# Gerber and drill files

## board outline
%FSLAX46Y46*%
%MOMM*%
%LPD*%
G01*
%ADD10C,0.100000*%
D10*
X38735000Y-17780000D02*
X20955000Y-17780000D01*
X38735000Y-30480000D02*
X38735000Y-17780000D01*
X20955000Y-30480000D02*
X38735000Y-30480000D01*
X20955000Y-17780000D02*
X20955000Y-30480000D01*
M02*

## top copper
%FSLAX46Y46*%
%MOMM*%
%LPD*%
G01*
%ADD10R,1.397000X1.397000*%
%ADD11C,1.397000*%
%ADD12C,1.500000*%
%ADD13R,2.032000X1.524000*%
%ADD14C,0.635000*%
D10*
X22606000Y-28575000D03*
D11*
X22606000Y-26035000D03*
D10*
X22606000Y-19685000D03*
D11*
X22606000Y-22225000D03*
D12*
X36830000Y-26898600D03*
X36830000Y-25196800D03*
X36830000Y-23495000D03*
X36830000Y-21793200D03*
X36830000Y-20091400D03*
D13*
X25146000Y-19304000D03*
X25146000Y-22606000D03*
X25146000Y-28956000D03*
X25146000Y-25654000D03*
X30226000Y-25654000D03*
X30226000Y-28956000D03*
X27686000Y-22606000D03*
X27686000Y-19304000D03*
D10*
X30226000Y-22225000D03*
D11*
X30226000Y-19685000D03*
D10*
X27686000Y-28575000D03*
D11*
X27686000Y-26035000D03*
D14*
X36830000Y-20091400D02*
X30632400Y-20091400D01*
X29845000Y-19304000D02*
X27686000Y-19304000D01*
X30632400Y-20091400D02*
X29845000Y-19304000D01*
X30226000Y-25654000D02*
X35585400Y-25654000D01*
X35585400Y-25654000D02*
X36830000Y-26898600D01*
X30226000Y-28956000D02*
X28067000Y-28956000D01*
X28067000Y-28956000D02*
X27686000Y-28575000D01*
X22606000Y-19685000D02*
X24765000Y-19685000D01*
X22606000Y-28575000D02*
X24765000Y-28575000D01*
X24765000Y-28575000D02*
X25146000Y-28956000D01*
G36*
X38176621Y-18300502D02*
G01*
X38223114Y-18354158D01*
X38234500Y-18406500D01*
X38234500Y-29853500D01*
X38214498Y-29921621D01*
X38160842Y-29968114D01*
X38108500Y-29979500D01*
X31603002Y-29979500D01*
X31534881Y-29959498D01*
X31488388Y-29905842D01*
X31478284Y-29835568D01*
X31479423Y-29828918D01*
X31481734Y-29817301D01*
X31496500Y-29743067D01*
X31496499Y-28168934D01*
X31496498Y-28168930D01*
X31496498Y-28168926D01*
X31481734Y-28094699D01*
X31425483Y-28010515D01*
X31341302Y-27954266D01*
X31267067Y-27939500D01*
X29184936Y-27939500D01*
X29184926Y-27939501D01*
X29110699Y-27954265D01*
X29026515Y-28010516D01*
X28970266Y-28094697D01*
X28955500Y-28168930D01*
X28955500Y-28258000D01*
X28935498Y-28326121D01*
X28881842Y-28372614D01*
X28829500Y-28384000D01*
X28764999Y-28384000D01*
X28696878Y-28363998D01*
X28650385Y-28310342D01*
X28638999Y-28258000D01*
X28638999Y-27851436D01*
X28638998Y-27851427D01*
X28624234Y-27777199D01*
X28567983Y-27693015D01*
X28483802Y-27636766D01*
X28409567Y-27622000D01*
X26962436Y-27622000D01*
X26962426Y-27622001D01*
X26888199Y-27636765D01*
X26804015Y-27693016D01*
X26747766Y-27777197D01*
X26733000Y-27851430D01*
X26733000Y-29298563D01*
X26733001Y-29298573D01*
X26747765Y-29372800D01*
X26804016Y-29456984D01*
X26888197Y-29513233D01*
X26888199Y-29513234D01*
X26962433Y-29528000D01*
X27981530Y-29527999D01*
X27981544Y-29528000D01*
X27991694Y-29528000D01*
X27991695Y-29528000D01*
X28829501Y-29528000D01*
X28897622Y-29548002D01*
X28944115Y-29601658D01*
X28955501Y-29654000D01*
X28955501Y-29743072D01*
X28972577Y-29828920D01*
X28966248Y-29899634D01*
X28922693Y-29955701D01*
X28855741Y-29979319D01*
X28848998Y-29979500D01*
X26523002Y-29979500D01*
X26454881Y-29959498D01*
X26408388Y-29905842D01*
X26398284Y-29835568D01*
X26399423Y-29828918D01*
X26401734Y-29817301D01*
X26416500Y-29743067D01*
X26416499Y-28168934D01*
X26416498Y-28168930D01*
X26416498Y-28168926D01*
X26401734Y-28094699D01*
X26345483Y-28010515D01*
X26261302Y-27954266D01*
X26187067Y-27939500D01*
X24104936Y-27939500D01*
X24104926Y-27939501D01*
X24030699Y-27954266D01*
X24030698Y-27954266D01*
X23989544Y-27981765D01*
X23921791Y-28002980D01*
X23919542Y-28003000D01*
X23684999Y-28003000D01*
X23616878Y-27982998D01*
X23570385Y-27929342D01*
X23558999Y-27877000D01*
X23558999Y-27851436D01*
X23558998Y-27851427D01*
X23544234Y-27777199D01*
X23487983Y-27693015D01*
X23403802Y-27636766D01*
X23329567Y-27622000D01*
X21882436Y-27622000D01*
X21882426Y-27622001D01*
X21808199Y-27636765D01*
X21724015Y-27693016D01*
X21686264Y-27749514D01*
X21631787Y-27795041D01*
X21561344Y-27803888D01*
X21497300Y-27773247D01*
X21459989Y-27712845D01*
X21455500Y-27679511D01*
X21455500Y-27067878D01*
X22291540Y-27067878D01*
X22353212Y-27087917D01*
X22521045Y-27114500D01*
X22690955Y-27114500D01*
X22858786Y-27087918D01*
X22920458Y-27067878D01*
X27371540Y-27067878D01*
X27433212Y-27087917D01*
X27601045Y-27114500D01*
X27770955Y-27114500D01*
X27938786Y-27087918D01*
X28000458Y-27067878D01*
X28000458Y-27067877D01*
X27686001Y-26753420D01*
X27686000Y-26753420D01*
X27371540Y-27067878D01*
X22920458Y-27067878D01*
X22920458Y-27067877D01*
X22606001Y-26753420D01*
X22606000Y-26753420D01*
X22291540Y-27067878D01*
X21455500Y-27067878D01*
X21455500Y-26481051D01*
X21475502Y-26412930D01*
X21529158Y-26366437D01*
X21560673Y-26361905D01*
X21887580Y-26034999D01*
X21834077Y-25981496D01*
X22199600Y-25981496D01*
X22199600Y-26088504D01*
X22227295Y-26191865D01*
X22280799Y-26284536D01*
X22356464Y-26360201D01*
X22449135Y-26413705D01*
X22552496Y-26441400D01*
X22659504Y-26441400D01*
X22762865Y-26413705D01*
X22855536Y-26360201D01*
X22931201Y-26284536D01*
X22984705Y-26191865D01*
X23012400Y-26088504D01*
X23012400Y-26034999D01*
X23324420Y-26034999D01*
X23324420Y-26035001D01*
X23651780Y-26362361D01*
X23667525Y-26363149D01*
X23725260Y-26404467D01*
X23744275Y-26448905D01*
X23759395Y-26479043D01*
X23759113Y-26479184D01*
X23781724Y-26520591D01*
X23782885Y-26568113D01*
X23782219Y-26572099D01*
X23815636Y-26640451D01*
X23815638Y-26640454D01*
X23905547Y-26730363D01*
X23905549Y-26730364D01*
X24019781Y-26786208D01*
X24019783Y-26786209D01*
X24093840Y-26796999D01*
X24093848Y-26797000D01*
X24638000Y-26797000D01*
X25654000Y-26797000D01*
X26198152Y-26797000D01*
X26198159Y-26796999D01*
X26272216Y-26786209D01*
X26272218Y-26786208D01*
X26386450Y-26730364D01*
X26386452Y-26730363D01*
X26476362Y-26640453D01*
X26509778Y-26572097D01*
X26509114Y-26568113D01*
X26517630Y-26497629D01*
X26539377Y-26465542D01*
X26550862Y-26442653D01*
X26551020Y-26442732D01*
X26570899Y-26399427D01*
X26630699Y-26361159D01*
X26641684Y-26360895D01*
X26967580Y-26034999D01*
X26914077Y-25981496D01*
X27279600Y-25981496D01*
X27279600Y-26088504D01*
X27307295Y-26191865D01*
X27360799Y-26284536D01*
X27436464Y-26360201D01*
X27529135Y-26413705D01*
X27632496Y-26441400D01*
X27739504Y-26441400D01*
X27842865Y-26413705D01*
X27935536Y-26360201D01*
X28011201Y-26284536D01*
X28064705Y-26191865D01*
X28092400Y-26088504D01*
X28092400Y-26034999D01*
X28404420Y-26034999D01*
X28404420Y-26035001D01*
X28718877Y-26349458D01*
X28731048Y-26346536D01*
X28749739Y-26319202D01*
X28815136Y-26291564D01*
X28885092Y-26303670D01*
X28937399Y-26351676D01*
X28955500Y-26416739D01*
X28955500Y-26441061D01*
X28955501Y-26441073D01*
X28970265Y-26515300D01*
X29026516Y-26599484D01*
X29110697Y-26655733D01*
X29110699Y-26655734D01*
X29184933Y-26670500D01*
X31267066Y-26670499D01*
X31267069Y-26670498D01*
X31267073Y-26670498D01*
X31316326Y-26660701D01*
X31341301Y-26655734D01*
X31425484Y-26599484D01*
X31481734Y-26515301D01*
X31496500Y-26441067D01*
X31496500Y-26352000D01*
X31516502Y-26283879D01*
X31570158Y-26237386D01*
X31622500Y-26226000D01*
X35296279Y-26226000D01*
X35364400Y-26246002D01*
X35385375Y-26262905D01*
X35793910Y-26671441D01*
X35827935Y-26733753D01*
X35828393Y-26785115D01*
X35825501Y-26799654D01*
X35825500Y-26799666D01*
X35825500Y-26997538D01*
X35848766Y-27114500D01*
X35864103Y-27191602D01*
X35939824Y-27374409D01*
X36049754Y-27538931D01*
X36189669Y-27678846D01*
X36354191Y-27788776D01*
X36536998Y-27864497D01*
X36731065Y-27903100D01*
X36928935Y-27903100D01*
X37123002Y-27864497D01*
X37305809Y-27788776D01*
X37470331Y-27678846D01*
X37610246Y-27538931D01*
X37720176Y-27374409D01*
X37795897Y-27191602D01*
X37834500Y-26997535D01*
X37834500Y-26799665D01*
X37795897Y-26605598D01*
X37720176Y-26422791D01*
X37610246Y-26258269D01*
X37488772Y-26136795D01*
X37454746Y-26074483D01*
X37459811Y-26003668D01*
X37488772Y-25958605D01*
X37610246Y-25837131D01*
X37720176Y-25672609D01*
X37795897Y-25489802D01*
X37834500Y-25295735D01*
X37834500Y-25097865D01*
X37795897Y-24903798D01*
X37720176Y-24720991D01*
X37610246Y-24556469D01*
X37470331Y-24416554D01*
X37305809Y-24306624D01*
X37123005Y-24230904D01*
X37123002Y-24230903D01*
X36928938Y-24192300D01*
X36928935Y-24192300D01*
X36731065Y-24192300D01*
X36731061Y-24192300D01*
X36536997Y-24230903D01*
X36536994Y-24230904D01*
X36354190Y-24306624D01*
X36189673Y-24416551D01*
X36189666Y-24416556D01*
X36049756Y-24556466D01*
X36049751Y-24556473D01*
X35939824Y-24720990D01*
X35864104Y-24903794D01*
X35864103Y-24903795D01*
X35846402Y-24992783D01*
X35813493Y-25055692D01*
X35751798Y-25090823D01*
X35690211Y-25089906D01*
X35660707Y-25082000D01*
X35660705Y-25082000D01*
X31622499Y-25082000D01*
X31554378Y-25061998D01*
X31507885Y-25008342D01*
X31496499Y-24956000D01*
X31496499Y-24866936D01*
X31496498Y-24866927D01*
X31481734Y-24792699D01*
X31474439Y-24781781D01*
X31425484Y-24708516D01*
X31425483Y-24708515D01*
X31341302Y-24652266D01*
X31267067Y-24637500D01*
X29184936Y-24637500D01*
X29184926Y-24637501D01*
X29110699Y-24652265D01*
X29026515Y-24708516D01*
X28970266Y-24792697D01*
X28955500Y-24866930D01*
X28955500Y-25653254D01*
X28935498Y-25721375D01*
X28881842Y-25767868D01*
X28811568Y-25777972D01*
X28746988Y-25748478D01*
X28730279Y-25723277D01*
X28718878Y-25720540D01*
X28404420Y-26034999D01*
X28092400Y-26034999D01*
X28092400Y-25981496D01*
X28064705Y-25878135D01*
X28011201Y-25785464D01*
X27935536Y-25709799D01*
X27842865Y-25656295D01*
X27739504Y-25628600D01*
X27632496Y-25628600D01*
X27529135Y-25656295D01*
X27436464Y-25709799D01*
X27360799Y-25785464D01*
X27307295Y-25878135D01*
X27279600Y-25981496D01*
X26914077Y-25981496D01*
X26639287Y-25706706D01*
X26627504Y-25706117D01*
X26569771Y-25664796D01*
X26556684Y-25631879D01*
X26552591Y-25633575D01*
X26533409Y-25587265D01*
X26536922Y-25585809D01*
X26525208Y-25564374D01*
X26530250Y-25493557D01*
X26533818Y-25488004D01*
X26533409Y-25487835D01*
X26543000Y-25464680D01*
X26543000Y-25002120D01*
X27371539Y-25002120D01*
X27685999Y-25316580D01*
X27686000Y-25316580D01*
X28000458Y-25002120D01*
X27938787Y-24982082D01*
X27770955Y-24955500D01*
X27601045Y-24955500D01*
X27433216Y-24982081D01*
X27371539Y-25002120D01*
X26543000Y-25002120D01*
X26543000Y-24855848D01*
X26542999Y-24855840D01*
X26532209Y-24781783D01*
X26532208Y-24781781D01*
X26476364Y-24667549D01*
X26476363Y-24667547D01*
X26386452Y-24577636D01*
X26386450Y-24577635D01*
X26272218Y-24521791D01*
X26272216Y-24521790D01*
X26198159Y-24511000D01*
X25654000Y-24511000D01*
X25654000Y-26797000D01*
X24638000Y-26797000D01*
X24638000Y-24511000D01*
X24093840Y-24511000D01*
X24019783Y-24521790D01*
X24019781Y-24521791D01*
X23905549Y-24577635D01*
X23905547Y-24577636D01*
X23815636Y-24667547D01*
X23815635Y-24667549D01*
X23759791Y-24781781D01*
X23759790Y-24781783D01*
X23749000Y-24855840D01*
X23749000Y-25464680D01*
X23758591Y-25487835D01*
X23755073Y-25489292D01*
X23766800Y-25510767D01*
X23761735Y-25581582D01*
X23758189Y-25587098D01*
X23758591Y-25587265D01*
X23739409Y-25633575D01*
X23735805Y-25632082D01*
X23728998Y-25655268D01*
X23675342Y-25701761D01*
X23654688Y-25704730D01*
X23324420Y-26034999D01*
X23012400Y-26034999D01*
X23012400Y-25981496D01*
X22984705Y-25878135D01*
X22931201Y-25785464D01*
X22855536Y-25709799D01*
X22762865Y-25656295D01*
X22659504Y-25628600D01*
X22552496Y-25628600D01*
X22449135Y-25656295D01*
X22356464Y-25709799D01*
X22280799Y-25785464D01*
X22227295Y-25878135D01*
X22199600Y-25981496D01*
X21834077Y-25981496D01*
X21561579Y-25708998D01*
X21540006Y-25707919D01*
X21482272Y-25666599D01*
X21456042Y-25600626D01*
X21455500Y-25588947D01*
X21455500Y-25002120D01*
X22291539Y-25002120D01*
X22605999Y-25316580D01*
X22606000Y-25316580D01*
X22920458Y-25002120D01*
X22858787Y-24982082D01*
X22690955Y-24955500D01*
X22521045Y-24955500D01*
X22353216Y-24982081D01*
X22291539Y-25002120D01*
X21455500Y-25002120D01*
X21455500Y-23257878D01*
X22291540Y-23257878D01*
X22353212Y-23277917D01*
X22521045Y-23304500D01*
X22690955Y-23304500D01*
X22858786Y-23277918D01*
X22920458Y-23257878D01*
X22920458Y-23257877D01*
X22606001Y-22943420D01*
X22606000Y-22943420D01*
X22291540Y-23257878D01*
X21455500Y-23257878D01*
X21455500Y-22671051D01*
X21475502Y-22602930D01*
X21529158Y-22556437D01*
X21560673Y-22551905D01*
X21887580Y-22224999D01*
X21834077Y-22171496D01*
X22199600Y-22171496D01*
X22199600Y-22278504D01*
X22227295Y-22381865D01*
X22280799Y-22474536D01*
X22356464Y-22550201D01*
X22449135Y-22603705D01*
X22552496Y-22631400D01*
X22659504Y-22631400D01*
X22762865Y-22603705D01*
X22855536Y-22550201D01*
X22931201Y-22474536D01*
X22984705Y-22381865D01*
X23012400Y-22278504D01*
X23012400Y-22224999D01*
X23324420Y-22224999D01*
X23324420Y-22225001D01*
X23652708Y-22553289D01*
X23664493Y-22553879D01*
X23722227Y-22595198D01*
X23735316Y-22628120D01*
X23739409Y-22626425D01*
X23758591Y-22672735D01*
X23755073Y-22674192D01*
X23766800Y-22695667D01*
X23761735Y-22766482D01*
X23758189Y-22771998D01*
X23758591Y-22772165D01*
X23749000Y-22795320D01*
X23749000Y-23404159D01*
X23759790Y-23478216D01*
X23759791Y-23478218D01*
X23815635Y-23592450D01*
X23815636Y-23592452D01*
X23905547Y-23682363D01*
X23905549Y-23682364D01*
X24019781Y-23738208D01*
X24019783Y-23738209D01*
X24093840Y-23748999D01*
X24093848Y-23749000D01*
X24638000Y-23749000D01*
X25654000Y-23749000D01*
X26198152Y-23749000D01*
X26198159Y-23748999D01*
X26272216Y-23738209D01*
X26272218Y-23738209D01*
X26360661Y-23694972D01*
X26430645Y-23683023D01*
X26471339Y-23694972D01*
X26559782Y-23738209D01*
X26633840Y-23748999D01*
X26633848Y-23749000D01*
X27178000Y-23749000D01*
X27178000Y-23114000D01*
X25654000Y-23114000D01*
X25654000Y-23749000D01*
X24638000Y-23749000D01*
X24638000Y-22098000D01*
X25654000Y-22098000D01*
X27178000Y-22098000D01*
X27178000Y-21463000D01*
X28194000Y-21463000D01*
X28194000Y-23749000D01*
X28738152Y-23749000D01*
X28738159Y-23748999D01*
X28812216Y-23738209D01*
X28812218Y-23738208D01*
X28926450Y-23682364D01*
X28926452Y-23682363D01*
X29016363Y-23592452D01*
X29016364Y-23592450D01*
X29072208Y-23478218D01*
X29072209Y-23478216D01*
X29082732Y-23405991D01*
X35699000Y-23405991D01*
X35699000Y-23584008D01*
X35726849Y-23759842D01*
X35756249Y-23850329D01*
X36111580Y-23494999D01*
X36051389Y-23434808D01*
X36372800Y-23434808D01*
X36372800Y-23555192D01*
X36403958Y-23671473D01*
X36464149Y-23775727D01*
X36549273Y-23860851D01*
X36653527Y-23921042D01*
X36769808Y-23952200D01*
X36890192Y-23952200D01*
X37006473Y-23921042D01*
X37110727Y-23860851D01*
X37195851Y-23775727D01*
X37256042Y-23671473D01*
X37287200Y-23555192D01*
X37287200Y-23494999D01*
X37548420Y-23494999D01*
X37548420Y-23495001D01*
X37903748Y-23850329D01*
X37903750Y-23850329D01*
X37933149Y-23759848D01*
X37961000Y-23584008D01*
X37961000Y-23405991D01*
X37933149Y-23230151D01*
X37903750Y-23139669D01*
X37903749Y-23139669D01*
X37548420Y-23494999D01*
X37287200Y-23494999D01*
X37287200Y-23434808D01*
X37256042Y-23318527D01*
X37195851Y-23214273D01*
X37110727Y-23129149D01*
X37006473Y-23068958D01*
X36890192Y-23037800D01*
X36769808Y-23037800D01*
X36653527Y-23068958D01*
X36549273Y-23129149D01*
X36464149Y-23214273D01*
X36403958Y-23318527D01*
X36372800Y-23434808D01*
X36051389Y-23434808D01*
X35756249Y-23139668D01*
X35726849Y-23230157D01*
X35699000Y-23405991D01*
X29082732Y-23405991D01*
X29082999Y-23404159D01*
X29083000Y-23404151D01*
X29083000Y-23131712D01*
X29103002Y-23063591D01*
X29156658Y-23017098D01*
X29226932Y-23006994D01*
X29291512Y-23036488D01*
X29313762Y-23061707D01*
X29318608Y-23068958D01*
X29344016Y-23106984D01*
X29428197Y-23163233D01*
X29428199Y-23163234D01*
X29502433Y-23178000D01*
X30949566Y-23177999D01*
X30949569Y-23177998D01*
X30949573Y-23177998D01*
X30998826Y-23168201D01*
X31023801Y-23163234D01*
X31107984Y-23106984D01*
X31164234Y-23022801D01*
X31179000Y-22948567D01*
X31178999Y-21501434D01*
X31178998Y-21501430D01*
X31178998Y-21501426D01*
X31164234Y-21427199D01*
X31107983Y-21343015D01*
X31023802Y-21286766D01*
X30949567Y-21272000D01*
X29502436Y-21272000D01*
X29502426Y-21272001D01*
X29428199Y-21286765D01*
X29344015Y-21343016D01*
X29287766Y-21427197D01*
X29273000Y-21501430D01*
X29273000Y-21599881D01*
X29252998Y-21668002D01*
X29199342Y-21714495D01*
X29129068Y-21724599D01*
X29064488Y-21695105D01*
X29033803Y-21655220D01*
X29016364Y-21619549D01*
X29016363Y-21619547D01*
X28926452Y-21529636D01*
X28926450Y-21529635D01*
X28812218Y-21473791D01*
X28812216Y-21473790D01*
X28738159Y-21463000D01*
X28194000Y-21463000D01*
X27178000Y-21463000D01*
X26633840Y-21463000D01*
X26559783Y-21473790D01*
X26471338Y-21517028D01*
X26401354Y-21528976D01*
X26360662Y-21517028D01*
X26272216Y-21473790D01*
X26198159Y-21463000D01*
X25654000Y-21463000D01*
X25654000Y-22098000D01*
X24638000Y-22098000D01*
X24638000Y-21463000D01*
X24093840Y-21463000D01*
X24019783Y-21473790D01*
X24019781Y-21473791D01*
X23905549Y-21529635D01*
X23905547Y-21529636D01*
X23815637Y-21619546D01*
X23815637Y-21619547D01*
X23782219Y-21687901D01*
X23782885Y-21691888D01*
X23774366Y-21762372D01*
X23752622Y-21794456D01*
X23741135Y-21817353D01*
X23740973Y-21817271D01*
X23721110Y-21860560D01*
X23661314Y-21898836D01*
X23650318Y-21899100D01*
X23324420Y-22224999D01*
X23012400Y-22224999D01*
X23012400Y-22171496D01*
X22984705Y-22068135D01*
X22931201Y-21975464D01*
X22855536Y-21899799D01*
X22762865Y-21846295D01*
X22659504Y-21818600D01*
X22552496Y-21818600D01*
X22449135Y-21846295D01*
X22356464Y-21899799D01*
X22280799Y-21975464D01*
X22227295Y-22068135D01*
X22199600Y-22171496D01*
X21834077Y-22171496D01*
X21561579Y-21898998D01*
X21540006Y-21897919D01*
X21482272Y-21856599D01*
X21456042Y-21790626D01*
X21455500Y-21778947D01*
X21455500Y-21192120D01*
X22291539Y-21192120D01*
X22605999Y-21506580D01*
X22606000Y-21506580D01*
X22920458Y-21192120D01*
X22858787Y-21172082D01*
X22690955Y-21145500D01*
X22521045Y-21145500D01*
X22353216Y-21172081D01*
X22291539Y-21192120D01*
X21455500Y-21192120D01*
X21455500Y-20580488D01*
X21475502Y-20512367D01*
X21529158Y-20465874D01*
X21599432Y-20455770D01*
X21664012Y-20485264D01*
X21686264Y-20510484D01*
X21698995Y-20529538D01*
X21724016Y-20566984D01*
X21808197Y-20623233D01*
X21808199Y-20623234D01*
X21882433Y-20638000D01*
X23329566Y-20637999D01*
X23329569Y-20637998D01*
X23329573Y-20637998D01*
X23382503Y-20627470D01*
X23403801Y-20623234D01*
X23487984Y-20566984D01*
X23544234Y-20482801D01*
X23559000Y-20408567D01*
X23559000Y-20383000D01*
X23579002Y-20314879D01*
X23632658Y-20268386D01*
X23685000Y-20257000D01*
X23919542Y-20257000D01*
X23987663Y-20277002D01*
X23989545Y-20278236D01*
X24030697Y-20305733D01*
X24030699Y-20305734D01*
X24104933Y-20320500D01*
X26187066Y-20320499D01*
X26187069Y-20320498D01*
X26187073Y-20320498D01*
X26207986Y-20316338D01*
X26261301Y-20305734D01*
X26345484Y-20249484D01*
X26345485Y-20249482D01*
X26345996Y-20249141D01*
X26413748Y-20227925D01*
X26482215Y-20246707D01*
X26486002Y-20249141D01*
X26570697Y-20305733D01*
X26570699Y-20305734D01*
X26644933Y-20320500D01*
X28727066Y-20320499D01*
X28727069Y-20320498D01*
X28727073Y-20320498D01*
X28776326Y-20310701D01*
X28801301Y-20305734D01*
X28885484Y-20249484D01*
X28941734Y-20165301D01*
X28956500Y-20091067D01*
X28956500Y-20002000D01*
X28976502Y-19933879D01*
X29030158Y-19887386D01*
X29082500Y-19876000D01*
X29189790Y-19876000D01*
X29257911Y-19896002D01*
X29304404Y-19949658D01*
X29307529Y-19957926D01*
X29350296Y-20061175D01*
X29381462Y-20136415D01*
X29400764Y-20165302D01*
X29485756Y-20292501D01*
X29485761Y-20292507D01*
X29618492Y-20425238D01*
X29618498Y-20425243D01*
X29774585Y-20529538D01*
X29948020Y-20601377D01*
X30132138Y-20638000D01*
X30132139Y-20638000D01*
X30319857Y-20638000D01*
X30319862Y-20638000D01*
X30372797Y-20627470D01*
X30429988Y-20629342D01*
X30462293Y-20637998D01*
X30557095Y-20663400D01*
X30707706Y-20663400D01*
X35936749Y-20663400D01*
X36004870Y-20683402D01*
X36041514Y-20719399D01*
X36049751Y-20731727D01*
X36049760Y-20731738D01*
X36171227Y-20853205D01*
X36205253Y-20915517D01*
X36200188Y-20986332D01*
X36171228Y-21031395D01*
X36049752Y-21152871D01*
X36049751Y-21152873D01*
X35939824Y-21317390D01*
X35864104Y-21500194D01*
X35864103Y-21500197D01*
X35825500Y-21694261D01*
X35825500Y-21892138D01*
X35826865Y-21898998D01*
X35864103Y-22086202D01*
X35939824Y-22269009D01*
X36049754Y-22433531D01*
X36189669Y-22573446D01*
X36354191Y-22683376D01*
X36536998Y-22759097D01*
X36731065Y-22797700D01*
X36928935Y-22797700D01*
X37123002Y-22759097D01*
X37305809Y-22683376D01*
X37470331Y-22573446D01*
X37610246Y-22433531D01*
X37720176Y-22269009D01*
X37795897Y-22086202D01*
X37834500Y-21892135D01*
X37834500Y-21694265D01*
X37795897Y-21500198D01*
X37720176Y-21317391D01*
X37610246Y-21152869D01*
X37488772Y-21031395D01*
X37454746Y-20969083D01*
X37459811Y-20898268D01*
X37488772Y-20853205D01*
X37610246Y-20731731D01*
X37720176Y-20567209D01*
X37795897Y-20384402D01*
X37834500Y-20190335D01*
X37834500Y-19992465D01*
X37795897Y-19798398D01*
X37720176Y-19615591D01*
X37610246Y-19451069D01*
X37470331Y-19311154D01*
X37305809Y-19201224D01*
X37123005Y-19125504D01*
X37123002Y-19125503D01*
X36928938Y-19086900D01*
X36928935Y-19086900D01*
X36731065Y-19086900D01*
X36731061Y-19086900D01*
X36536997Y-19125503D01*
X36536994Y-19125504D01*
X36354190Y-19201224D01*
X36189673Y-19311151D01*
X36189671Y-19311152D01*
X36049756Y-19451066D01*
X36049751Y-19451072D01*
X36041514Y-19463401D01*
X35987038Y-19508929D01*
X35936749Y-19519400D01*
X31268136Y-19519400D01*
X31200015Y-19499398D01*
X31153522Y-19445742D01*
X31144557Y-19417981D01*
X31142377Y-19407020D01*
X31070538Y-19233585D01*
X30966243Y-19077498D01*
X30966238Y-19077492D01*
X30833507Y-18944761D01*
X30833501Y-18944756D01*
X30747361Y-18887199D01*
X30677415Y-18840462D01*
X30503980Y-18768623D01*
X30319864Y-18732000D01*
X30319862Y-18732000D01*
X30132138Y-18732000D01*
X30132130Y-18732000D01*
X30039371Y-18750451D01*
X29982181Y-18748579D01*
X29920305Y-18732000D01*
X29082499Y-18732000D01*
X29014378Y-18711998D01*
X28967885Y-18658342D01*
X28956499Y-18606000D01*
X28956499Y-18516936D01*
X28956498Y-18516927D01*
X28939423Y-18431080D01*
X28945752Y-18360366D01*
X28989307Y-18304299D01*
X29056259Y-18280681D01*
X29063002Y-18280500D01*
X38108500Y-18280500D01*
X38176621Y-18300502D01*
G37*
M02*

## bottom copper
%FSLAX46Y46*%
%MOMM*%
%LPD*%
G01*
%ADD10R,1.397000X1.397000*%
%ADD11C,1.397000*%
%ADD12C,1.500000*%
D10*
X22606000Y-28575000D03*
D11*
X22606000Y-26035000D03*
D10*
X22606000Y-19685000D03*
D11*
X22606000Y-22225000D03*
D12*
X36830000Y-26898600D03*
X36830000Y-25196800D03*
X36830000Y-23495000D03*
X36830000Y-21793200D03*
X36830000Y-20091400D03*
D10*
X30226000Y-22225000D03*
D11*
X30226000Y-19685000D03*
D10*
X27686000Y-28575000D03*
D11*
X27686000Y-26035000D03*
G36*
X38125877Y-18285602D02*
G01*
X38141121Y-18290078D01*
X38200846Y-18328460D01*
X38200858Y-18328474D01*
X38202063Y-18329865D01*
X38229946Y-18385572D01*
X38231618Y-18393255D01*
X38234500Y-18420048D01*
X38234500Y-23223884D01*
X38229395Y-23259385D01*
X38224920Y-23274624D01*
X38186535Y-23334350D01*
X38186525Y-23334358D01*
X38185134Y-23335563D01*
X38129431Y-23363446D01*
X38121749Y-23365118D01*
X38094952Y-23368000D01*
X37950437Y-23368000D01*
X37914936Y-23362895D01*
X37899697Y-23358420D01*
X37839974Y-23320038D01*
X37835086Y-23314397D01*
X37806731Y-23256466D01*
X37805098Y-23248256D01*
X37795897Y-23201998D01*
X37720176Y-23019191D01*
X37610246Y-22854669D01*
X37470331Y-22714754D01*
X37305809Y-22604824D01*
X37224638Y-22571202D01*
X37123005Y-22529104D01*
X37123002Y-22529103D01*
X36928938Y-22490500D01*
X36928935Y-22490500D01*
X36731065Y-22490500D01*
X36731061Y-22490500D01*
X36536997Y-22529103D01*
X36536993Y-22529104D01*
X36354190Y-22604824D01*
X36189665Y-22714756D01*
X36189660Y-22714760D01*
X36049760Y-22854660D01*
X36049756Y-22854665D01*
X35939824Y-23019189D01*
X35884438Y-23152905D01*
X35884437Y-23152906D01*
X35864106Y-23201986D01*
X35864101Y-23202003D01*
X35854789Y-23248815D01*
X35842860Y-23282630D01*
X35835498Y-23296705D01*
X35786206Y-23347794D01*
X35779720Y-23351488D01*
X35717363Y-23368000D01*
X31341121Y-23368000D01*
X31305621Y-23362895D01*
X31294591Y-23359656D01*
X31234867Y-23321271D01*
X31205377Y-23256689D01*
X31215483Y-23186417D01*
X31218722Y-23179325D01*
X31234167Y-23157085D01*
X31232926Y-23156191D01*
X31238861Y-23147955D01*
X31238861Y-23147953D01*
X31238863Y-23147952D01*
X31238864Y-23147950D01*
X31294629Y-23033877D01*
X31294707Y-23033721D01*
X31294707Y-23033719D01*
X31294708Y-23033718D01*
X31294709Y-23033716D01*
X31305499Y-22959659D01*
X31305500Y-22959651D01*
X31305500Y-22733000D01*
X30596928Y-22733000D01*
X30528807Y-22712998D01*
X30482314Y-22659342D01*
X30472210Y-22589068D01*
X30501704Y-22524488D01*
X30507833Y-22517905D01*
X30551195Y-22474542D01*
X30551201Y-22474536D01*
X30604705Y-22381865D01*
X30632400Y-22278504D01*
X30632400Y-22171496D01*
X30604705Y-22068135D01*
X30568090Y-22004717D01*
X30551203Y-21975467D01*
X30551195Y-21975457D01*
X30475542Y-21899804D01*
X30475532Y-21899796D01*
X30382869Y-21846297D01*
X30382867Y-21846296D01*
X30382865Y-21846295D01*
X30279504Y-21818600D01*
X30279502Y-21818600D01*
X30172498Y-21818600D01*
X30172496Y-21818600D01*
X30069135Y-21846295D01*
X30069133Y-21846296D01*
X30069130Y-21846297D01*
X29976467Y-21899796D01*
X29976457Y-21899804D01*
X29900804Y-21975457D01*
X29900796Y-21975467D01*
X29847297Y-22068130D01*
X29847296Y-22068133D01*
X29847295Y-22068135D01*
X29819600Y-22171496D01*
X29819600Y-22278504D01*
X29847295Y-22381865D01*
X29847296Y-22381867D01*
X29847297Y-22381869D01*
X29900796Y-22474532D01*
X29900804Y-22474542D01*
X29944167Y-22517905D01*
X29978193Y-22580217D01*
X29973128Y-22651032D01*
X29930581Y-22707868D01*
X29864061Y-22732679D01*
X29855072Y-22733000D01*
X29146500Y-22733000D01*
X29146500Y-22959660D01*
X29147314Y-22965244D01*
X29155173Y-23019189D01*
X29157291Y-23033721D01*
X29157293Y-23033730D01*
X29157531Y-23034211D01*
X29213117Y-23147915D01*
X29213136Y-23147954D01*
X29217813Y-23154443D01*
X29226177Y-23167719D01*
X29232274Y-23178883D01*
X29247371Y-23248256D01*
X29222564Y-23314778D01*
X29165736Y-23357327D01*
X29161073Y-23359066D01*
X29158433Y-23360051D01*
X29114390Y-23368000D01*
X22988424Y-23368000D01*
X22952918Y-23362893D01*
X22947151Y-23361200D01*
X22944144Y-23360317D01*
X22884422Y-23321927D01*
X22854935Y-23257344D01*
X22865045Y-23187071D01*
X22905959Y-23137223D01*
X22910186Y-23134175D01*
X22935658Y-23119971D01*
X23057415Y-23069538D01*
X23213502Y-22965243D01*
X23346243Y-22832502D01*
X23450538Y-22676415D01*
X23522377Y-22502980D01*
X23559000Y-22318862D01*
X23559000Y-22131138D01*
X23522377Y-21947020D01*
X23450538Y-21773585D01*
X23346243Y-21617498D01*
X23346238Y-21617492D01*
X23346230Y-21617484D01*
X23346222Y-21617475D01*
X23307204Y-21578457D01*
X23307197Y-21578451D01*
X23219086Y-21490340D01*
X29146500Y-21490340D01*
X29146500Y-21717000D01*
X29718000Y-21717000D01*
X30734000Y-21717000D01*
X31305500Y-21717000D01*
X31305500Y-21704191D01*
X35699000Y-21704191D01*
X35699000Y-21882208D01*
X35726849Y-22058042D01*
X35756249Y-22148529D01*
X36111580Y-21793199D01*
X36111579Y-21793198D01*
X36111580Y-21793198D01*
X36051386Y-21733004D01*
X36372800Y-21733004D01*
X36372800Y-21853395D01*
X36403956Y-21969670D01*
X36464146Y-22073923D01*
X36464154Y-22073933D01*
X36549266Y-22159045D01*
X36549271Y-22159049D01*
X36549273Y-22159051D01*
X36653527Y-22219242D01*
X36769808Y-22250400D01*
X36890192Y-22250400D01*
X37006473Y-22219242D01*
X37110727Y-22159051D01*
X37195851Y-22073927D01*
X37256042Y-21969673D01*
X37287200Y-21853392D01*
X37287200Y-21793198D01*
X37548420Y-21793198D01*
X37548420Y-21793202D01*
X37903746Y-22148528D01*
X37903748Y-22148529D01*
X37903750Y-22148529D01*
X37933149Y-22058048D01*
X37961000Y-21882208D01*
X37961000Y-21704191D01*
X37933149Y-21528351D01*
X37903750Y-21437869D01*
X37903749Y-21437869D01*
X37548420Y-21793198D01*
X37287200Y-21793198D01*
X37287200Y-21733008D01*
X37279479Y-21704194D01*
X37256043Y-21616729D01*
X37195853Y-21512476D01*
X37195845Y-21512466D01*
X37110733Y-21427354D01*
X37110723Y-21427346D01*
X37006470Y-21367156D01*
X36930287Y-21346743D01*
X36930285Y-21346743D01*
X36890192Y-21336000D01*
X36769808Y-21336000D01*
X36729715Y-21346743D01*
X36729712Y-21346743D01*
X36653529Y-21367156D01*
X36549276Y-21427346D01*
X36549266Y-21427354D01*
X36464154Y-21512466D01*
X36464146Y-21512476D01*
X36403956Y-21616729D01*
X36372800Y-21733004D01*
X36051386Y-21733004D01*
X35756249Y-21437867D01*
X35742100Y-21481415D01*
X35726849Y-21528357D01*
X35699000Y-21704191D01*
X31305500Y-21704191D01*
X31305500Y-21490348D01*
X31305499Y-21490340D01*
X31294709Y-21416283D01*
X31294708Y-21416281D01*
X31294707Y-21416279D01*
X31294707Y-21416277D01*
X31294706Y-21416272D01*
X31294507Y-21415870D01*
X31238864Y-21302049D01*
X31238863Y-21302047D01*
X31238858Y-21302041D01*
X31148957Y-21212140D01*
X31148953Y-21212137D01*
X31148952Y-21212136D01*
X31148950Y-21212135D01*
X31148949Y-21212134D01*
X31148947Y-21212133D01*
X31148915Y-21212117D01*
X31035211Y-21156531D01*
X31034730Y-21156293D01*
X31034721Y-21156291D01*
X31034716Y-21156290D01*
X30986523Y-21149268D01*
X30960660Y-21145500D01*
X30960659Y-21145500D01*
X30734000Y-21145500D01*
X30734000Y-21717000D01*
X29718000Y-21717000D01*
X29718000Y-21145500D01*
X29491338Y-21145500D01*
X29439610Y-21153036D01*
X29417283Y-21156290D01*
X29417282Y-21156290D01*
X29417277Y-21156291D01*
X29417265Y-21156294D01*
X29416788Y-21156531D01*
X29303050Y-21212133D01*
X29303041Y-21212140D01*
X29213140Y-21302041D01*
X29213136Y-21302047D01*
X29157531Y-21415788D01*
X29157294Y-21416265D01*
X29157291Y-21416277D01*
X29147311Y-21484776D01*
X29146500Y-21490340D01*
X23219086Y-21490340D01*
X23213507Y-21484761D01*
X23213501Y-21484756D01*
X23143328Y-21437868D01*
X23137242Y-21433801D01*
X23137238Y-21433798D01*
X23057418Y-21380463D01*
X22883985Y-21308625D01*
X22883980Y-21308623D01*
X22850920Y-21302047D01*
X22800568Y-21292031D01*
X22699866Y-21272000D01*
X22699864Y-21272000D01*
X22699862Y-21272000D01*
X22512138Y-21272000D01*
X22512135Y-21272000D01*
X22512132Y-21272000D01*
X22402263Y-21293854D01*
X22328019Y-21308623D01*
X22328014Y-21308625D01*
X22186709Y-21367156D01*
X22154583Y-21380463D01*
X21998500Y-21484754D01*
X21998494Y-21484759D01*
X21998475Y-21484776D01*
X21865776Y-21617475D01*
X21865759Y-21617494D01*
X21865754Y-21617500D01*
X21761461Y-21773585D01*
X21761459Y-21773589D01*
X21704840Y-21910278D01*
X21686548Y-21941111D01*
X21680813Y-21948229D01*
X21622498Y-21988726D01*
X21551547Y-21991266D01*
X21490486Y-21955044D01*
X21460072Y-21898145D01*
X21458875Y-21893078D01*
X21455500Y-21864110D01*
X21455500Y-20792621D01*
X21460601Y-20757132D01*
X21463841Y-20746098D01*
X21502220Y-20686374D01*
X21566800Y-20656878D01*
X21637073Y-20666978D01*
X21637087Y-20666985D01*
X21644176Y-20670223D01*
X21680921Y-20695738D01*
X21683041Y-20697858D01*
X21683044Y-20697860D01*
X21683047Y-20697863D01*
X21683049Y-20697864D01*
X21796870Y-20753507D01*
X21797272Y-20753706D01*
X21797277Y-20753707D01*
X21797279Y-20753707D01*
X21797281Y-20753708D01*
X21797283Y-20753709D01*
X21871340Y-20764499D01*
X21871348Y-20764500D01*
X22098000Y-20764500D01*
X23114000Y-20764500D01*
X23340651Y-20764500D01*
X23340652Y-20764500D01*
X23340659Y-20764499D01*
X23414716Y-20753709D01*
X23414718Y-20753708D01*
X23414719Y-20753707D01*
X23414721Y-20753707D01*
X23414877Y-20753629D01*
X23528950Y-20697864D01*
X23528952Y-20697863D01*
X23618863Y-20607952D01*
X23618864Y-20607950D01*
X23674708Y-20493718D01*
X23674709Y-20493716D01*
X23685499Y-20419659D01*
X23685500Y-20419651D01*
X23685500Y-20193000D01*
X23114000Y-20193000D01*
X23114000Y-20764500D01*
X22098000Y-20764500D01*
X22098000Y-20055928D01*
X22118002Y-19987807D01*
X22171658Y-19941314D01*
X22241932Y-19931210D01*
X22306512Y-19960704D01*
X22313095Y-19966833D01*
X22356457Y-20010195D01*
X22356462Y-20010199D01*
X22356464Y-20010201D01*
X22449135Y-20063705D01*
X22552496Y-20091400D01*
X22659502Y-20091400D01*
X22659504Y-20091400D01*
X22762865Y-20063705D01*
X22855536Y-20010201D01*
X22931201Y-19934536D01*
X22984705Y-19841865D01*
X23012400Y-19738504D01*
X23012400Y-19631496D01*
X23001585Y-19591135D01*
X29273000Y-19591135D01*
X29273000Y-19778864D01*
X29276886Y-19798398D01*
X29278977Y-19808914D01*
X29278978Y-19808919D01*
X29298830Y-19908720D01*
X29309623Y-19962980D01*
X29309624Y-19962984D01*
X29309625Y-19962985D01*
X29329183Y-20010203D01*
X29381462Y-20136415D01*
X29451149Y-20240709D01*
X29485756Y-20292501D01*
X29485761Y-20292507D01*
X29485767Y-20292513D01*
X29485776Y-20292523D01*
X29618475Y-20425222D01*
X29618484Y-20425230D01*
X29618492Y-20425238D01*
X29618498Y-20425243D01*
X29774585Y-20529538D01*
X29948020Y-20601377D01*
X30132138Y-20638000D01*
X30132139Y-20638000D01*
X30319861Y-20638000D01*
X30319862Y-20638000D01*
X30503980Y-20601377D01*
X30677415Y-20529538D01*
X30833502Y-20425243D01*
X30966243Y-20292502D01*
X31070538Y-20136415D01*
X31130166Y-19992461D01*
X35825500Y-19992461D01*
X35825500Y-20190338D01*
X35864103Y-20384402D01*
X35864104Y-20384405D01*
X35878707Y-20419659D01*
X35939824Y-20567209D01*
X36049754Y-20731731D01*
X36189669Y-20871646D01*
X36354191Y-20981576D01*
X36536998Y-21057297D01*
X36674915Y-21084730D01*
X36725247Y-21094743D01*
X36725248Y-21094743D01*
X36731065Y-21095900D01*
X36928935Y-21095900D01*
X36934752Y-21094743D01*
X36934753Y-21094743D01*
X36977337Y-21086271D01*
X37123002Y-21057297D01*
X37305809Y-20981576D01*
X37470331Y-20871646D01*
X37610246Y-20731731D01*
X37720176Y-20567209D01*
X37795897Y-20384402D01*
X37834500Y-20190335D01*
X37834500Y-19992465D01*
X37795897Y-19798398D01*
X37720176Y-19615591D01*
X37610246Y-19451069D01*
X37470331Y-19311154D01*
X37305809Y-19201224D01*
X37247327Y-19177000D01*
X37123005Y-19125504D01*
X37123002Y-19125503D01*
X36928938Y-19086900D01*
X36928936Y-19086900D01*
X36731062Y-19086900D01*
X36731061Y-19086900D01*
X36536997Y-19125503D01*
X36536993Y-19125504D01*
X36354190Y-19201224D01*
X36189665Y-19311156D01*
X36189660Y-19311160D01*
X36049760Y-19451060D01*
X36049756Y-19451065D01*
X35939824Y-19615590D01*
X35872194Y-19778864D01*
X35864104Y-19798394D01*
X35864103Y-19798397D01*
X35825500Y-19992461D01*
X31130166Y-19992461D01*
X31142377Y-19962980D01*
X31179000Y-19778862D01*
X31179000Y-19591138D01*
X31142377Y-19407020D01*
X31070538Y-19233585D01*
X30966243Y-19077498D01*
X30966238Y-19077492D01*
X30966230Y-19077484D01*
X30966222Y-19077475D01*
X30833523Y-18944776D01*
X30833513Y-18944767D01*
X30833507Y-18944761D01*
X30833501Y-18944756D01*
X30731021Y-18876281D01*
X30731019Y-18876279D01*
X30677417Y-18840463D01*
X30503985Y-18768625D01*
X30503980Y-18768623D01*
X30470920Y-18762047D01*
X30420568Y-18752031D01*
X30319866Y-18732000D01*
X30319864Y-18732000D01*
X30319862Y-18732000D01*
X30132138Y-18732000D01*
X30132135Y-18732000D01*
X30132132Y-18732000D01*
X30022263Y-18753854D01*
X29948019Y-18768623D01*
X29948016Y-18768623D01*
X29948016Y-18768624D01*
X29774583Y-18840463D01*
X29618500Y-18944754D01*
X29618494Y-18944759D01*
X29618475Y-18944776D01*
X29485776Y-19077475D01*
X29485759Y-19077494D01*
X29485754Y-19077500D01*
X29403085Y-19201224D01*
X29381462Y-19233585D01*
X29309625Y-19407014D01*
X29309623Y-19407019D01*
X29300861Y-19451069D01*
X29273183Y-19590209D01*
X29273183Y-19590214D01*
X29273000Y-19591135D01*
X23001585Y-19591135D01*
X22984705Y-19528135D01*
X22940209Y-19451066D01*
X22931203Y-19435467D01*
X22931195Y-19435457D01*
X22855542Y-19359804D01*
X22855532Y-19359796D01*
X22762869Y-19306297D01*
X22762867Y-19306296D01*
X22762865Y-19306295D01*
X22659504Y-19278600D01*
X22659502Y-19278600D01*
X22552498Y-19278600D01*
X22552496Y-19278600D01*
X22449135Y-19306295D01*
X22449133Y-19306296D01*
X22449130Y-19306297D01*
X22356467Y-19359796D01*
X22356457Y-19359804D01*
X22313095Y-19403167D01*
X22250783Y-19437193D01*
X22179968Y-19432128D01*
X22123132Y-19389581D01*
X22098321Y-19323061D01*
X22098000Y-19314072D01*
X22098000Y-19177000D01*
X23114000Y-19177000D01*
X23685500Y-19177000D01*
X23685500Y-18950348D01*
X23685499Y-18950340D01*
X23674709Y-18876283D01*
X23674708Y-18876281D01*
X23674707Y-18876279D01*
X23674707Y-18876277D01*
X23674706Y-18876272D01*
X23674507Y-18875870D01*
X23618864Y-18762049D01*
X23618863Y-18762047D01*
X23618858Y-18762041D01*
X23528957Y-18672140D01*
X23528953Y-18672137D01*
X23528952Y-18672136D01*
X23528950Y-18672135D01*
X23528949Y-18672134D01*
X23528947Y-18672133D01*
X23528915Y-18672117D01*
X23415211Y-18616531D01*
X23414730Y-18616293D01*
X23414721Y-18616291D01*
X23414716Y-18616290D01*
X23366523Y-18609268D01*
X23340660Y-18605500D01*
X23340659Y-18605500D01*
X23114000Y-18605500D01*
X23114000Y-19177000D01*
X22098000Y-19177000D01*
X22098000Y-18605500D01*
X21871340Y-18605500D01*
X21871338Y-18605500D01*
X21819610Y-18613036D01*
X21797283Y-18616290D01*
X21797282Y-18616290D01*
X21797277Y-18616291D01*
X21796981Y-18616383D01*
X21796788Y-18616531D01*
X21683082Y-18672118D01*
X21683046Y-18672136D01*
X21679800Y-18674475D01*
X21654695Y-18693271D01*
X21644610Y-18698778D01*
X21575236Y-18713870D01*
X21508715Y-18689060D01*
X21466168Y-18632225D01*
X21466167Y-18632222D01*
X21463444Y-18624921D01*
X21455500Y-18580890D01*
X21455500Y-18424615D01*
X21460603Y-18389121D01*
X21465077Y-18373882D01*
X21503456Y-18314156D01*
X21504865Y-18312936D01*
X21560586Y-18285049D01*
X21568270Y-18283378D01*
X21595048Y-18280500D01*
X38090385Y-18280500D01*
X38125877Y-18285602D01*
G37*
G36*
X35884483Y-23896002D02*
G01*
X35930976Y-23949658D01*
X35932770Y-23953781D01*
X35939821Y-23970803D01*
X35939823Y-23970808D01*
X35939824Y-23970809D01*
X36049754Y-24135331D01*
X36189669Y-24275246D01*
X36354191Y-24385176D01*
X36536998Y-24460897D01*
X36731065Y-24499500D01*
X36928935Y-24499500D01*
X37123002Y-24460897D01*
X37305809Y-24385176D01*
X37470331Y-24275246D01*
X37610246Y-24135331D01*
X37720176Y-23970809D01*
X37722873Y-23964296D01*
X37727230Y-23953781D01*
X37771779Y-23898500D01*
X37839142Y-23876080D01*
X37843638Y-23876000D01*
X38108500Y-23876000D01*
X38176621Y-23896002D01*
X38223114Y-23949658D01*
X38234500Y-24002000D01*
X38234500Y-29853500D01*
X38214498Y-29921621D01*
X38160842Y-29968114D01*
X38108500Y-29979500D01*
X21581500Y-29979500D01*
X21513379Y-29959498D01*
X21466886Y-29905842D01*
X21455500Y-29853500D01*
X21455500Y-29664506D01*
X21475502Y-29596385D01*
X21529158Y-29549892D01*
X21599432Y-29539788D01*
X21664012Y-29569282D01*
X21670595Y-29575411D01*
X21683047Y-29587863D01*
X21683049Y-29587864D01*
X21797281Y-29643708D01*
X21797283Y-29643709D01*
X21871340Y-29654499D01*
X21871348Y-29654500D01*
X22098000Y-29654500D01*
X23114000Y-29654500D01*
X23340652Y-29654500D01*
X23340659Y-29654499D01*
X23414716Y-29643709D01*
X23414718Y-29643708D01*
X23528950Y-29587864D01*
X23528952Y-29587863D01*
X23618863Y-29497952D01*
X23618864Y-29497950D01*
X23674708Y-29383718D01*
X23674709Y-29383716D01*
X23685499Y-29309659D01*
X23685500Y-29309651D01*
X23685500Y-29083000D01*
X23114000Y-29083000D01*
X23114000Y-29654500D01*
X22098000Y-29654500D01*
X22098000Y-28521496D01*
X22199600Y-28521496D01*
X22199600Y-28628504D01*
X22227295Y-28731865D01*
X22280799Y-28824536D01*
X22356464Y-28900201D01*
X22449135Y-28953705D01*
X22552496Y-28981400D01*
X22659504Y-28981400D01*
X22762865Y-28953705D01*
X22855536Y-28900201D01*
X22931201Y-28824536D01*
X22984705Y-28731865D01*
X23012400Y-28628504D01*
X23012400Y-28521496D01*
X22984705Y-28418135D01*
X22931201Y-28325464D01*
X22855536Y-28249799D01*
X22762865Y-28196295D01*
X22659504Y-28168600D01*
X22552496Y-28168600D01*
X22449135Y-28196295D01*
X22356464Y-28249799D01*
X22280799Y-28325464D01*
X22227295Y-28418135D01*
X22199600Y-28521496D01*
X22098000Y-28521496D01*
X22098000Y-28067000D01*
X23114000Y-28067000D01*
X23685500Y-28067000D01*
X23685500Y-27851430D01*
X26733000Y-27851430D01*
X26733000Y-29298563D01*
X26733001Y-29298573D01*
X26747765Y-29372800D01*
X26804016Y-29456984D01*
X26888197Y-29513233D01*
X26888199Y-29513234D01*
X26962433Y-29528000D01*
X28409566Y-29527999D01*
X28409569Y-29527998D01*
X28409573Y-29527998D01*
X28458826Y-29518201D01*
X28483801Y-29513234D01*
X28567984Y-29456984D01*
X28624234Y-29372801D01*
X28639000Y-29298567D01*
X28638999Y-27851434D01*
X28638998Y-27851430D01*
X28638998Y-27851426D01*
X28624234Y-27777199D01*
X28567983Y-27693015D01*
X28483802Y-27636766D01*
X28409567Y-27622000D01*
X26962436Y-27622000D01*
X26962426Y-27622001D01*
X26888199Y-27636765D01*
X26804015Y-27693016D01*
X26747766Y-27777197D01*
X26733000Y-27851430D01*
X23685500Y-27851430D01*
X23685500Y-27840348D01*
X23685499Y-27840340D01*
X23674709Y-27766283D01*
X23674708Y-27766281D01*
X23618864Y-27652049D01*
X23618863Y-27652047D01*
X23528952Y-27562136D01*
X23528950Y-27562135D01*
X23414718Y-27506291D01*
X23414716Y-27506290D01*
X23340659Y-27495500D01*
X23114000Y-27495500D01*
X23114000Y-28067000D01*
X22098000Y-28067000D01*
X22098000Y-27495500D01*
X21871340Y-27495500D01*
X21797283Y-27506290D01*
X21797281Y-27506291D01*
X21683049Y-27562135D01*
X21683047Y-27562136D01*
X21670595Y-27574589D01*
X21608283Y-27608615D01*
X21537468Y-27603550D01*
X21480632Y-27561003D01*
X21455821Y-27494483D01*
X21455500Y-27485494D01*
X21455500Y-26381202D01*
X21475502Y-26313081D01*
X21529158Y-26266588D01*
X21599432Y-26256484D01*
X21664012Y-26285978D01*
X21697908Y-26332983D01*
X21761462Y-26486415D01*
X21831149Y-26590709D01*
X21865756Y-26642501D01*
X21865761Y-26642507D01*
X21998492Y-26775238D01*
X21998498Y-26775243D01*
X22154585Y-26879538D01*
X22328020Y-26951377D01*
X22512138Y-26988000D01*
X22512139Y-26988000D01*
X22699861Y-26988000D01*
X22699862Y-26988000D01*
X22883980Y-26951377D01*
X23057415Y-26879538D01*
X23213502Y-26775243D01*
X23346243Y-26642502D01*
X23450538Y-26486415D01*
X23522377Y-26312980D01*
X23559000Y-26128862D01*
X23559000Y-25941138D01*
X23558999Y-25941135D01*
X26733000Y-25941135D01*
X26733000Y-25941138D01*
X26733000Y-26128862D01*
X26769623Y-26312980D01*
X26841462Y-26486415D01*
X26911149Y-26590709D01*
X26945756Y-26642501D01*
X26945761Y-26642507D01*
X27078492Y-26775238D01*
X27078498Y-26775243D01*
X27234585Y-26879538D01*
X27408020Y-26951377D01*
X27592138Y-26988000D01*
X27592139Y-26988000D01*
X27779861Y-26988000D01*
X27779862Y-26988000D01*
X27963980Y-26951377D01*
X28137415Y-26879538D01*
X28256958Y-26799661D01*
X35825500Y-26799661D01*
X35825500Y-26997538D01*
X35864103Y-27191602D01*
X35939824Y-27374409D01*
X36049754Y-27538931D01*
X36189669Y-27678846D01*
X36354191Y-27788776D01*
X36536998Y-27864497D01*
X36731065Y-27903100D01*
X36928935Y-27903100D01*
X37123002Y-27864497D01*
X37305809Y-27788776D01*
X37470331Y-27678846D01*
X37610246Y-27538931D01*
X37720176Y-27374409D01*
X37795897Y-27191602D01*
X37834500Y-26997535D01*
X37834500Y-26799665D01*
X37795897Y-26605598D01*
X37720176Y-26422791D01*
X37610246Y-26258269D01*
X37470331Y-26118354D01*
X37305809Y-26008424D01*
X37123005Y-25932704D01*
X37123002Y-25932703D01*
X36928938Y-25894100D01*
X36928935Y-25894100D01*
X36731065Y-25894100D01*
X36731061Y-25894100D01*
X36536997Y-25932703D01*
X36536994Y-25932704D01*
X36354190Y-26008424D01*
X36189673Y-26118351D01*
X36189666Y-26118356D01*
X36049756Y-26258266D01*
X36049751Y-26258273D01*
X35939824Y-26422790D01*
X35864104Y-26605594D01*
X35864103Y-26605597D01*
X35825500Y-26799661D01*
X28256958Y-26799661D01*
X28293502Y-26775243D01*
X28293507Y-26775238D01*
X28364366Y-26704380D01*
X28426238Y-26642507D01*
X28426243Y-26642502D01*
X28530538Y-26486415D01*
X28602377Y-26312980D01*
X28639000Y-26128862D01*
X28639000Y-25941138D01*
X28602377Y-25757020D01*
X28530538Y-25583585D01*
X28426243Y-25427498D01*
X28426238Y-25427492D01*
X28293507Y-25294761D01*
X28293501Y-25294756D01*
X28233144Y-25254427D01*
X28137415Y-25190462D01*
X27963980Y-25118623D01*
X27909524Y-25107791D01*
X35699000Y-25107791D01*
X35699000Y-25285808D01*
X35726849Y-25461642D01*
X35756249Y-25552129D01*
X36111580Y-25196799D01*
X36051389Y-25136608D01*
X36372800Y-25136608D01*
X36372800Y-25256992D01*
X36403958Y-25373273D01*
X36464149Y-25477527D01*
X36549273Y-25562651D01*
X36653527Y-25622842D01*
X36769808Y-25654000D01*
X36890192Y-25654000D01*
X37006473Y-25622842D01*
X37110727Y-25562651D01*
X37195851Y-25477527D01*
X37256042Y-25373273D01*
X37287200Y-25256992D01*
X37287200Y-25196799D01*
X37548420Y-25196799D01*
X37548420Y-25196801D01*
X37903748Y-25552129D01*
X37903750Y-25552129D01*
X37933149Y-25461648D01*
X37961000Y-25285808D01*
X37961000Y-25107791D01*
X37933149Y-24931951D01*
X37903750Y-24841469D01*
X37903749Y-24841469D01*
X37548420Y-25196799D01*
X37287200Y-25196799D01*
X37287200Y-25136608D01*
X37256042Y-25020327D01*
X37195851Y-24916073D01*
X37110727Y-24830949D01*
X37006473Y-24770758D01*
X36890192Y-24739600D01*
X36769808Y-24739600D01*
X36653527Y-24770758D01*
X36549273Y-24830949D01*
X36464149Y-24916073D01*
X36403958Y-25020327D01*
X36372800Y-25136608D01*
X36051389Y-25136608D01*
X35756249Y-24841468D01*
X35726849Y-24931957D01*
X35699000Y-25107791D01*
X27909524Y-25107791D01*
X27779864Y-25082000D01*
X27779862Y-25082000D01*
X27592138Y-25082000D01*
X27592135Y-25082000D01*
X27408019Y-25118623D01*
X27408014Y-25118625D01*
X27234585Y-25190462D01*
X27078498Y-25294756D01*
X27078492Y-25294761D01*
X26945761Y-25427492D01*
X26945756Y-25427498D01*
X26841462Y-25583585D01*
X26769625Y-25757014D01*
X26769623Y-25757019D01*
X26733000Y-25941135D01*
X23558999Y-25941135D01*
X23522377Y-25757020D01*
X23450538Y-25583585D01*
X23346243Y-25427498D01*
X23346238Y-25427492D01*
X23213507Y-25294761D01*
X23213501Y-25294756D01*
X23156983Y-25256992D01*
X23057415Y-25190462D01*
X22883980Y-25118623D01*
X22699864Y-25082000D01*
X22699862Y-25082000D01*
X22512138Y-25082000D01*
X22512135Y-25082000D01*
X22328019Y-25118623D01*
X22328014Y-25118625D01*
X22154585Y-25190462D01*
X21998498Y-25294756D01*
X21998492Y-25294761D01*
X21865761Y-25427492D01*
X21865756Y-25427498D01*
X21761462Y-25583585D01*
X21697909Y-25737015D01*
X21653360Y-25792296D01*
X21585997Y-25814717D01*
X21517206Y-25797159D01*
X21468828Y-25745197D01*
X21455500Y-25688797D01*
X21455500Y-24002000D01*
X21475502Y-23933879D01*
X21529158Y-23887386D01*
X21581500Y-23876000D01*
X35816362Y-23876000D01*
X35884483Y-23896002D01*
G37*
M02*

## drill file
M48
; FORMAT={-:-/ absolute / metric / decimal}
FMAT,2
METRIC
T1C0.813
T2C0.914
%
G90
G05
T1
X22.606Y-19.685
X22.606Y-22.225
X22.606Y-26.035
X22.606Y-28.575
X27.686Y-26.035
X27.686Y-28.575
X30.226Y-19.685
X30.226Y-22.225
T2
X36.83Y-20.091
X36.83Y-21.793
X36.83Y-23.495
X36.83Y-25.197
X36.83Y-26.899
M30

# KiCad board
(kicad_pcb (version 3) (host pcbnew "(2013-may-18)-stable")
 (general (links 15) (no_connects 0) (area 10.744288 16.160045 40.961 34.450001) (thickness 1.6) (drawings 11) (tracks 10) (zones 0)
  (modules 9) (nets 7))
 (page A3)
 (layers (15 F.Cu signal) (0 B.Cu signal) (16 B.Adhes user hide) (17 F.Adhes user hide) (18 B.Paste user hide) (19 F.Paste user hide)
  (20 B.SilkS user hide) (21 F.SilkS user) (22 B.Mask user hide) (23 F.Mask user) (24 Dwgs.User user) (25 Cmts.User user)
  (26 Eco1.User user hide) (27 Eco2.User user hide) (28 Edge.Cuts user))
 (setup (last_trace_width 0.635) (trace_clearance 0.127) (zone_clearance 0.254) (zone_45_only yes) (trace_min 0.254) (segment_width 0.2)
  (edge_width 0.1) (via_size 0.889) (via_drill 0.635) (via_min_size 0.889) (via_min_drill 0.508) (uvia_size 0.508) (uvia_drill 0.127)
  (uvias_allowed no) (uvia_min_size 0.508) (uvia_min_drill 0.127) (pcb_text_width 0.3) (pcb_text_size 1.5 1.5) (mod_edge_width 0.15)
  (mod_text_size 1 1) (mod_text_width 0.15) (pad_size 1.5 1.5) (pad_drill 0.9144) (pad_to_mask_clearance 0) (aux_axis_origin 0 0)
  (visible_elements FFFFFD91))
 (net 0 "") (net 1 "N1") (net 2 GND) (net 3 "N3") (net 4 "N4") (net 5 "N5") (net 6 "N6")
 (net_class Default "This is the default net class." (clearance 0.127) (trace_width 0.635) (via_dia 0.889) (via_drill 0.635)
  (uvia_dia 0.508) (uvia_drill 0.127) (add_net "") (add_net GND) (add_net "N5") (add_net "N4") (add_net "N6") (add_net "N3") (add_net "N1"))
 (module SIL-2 (layer F.Cu) (at 22.606 27.305 90)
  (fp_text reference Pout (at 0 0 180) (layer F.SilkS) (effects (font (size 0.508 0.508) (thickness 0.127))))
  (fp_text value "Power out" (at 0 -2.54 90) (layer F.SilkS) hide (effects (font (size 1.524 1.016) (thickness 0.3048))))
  (pad 1 thru_hole rect (at -1.27 0 90) (size 1.397 1.397) (drill 0.8128) (layers *.Cu *.Mask F.SilkS) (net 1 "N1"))
  (pad 2 thru_hole circle (at 1.27 0 90) (size 1.397 1.397) (drill 0.8128) (layers *.Cu *.Mask F.SilkS) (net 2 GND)))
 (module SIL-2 (layer F.Cu) (at 22.606 20.955 270)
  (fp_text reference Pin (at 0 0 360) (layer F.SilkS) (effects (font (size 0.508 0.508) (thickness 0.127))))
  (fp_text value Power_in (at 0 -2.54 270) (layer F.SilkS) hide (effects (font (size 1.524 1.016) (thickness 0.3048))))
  (pad 1 thru_hole rect (at -1.27 0 270) (size 1.397 1.397) (drill 0.8128) (layers *.Cu *.Mask F.SilkS) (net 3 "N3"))
  (pad 2 thru_hole circle (at 1.27 0 270) (size 1.397 1.397) (drill 0.8128) (layers *.Cu *.Mask F.SilkS) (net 2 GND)))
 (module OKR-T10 (layer F.Cu) (at 36.83 23.495 90)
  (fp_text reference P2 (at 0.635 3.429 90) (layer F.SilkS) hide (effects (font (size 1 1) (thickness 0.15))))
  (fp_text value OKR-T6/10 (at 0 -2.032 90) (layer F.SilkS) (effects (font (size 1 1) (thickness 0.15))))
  (pad 5 thru_hole circle (at -3.4036 0 90) (size 1.5 1.5) (drill 0.9144) (layers *.Cu *.Mask F.SilkS) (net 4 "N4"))
  (pad 4 thru_hole circle (at -1.7018 0 90) (size 1.5 1.5) (drill 0.9144) (layers *.Cu *.Mask F.SilkS) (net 1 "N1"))
  (pad 3 thru_hole circle (at 0 0 90) (size 1.5 1.5) (drill 0.9144) (layers *.Cu *.Mask F.SilkS) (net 2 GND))
  (pad 2 thru_hole circle (at 1.7018 0 90) (size 1.5 1.5) (drill 0.9144) (layers *.Cu *.Mask F.SilkS) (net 3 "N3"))
  (pad 1 thru_hole circle (at 3.4036 0 90) (size 1.5 1.5) (drill 0.9144) (layers *.Cu *.Mask F.SilkS) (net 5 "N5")))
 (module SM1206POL (layer F.Cu) (at 25.146 20.955 270)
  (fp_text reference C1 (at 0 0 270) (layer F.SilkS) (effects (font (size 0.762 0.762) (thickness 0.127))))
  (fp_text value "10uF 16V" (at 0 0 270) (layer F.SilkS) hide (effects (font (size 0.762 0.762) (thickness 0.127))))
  (pad 1 smd rect (at -1.651 0 270) (size 1.524 2.032) (layers F.Cu F.Paste F.Mask) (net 3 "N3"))
  (pad 2 smd rect (at 1.651 0 270) (size 1.524 2.032) (layers F.Cu F.Paste F.Mask) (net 2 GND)))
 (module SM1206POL (layer F.Cu) (at 25.146 27.305 90)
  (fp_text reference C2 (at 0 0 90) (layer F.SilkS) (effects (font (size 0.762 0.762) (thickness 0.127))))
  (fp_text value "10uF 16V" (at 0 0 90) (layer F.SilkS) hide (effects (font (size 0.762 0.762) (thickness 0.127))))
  (pad 1 smd rect (at -1.651 0 90) (size 1.524 2.032) (layers F.Cu F.Paste F.Mask) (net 1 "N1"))
  (pad 2 smd rect (at 1.651 0 90) (size 1.524 2.032) (layers F.Cu F.Paste F.Mask) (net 2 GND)))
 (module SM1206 (layer F.Cu) (at 30.226 27.305 270)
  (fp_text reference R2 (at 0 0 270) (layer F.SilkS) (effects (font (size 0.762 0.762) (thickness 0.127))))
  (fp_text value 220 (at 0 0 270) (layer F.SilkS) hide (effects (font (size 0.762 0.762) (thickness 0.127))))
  (pad 1 smd rect (at -1.651 0 270) (size 1.524 2.032) (layers F.Cu F.Paste F.Mask) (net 4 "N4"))
  (pad 2 smd rect (at 1.651 0 270) (size 1.524 2.032) (layers F.Cu F.Paste F.Mask) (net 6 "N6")))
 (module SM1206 (layer F.Cu) (at 27.686 20.955 90)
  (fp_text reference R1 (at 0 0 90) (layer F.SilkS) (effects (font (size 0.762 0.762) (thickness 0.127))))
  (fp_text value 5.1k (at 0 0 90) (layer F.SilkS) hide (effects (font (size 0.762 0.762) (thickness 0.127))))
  (pad 1 smd rect (at -1.651 0 90) (size 1.524 2.032) (layers F.Cu F.Paste F.Mask) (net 2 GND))
  (pad 2 smd rect (at 1.651 0 90) (size 1.524 2.032) (layers F.Cu F.Paste F.Mask) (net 5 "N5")))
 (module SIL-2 (layer F.Cu) (at 30.226 20.955 90)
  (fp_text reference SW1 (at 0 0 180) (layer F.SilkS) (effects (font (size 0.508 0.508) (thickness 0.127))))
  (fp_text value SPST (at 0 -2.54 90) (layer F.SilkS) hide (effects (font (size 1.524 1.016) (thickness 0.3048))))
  (pad 1 thru_hole rect (at -1.27 0 90) (size 1.397 1.397) (drill 0.8128) (layers *.Cu *.Mask F.SilkS) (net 3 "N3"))
  (pad 2 thru_hole circle (at 1.27 0 90) (size 1.397 1.397) (drill 0.8128) (layers *.Cu *.Mask F.SilkS) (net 5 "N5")))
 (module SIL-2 (layer F.Cu) (at 27.686 27.305 90)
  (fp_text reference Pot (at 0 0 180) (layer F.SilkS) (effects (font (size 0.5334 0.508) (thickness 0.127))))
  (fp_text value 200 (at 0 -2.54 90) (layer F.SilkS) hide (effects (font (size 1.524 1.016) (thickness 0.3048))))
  (pad 1 thru_hole rect (at -1.27 0 90) (size 1.397 1.397) (drill 0.8128) (layers *.Cu *.Mask F.SilkS) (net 6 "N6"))
  (pad 2 thru_hole circle (at 1.27 0 90) (size 1.397 1.397) (drill 0.8128) (layers *.Cu *.Mask F.SilkS) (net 2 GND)))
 (gr_line (start 38.735 17.78) (end 20.955 17.78) (angle 90) (layer Edge.Cuts) (width 0.1))
 (gr_line (start 38.735 30.48) (end 38.735 17.78) (angle 90) (layer Edge.Cuts) (width 0.1))
 (gr_line (start 20.955 30.48) (end 38.735 30.48) (angle 90) (layer Edge.Cuts) (width 0.1))
 (gr_line (start 20.955 17.78) (end 20.955 30.48) (angle 90) (layer Edge.Cuts) (width 0.1))
 (segment (start 36.83 20.0914) (end 30.6324 20.0914) (width 0.635) (layer F.Cu) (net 5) (status 10))
 (segment (start 29.845 19.304) (end 27.686 19.304) (width 0.635) (layer F.Cu) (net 5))
 (segment (start 30.6324 20.0914) (end 29.845 19.304) (width 0.635) (layer F.Cu) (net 5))
 (segment (start 30.226 25.654) (end 35.5854 25.654) (width 0.635) (layer F.Cu) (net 4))
 (segment (start 35.5854 25.654) (end 36.83 26.8986) (width 0.635) (layer F.Cu) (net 4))
 (segment (start 30.226 28.956) (end 28.067 28.956) (width 0.635) (layer F.Cu) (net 6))
 (segment (start 28.067 28.956) (end 27.686 28.575) (width 0.635) (layer F.Cu) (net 6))
 (segment (start 22.606 19.685) (end 24.765 19.685) (width 0.635) (layer F.Cu) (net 3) (status 10))
 (segment (start 22.606 28.575) (end 24.765 28.575) (width 0.635) (layer F.Cu) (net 1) (status 10))
 (segment (start 24.765 28.575) (end 25.146 28.956) (width 0.635) (layer F.Cu) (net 1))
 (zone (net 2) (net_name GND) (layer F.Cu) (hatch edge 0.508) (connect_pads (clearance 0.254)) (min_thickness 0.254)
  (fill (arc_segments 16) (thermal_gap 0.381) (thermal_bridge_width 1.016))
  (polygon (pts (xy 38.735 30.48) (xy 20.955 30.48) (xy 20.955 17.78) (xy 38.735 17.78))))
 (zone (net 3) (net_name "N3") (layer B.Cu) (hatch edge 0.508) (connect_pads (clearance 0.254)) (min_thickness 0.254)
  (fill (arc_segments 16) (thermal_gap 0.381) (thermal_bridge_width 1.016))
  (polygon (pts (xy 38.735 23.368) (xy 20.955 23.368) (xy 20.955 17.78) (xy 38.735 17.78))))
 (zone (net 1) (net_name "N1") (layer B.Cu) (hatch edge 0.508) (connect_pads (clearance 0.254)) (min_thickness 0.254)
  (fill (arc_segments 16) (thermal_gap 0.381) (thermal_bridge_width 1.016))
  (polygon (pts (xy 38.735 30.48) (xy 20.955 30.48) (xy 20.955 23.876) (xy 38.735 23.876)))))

